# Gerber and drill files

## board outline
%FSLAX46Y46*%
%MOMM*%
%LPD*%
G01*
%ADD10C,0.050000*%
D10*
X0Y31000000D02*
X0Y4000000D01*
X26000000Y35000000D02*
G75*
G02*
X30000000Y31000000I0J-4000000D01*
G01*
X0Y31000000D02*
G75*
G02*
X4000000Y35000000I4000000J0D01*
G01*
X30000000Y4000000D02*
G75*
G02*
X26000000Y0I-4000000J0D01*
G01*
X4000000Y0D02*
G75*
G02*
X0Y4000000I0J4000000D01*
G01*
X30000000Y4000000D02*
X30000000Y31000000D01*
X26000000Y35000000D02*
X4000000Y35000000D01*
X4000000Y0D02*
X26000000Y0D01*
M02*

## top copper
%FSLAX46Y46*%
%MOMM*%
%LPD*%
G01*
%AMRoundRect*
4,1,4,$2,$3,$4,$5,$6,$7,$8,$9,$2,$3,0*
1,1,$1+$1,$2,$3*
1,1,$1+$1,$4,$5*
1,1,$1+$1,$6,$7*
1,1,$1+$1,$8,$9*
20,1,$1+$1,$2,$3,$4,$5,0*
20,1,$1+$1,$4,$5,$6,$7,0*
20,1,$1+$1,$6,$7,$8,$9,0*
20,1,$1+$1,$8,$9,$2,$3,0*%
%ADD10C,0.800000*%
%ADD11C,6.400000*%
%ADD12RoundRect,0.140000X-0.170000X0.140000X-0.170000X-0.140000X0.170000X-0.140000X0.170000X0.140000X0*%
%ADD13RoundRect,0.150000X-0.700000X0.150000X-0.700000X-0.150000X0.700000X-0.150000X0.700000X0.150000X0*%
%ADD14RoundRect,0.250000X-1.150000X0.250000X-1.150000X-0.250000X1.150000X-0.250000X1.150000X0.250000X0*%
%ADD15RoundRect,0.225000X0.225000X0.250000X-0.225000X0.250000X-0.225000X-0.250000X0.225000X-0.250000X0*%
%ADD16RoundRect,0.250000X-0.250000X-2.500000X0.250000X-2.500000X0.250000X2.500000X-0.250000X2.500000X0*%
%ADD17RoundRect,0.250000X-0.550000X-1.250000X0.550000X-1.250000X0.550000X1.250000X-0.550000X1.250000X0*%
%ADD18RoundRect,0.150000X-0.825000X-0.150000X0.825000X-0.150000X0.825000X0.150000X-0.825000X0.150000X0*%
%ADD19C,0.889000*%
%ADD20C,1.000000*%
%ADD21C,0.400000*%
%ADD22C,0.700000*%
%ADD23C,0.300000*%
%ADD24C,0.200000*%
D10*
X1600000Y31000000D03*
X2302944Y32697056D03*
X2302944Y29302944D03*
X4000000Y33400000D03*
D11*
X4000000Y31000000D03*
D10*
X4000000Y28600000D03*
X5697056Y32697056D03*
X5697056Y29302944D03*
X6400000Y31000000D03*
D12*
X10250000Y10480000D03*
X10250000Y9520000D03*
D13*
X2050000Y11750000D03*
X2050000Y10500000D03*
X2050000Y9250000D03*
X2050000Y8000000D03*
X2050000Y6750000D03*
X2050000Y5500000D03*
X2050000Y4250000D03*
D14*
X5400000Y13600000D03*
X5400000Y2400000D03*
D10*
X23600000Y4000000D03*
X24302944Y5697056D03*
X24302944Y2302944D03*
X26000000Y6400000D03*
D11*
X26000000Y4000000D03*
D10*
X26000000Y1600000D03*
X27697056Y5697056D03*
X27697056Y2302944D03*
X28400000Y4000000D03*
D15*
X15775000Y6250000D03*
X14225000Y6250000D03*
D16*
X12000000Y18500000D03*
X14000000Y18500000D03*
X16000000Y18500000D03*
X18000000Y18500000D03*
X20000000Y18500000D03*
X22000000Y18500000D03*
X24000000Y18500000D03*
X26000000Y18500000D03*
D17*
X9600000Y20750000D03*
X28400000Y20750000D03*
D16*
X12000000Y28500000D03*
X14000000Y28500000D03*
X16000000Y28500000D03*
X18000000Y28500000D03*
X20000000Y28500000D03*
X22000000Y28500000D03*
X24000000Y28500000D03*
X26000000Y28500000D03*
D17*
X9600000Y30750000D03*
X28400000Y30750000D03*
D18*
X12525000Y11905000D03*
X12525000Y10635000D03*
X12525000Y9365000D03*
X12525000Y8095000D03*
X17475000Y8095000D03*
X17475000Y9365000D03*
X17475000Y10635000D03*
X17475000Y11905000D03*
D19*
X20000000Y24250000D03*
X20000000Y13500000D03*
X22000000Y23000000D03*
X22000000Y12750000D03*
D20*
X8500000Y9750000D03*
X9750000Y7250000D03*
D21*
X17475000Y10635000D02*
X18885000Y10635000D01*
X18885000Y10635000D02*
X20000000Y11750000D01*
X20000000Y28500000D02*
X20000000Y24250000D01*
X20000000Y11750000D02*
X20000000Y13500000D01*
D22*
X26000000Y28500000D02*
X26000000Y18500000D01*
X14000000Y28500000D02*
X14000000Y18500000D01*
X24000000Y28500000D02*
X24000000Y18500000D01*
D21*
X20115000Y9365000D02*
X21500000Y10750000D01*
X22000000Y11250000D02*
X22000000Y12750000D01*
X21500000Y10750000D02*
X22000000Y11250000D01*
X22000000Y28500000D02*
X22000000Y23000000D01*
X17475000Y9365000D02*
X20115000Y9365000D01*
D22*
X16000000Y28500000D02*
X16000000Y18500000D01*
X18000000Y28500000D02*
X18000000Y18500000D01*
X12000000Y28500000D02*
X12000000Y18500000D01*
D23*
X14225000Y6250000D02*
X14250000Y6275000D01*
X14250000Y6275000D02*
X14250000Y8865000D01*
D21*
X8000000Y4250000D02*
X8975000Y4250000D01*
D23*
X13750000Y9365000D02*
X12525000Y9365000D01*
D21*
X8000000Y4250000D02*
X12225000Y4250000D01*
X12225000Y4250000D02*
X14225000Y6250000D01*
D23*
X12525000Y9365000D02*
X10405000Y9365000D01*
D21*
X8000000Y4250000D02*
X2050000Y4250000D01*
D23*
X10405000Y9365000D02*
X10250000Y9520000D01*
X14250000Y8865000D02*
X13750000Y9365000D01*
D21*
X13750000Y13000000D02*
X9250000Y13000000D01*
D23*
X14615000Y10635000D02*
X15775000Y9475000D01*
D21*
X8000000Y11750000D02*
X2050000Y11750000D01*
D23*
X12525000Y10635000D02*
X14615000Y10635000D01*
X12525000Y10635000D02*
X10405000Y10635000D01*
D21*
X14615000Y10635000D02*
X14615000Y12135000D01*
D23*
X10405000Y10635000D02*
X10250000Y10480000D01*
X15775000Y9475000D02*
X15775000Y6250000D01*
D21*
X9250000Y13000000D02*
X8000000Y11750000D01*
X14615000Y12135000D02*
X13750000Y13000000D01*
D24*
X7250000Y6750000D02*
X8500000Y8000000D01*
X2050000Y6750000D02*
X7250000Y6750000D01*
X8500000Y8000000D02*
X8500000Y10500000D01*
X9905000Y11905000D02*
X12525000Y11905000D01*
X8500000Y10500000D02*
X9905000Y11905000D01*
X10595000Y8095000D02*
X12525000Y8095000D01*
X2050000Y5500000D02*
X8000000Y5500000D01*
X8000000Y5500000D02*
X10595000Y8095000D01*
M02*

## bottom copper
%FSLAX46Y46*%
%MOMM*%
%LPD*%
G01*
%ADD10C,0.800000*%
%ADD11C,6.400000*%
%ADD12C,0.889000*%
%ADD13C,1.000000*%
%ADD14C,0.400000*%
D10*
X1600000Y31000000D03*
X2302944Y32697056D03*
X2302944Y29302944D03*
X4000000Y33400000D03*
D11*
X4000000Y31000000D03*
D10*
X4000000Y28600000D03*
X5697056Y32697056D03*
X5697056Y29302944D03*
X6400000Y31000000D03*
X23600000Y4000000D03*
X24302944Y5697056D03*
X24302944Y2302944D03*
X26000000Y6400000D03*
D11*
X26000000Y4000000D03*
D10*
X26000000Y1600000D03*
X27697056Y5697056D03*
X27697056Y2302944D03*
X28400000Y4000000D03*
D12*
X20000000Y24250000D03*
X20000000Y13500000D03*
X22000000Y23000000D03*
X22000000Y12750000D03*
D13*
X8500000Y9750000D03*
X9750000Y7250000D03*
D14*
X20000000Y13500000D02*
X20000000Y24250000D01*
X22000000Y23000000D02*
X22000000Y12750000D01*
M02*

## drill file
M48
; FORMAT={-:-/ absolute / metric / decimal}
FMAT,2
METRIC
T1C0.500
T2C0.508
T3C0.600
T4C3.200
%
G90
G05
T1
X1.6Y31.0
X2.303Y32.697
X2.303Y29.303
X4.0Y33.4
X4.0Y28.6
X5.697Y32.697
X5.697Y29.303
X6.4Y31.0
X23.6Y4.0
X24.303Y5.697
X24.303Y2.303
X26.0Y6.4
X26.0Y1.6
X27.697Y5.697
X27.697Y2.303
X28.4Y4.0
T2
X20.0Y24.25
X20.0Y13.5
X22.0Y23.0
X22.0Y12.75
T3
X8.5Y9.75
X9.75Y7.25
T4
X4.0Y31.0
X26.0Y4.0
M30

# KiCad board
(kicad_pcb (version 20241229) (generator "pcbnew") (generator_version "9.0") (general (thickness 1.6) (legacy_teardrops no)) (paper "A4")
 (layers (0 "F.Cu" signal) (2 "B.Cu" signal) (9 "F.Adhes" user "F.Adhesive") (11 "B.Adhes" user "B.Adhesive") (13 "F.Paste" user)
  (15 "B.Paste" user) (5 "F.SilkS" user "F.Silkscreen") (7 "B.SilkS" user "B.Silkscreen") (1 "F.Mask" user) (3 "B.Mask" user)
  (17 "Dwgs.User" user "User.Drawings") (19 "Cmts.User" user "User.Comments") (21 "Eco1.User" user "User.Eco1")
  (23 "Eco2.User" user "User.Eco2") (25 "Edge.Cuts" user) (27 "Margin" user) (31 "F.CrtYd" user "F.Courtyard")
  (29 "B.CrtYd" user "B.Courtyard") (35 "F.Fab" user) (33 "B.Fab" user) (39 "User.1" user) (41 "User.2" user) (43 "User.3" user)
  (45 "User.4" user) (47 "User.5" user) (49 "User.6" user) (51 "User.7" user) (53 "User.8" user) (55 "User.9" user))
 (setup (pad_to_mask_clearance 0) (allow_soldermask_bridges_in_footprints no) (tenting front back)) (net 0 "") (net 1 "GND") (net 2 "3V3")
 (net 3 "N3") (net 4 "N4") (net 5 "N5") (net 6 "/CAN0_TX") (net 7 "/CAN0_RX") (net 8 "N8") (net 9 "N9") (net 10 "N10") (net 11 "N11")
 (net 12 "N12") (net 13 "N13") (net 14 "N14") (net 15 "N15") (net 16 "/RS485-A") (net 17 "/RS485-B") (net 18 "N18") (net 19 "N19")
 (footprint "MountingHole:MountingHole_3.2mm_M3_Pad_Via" (layer "F.Cu") (at 4 -31)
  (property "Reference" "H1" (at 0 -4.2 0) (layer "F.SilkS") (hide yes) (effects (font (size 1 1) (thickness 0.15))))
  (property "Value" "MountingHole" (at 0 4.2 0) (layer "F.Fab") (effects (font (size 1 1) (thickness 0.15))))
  (pad "1" thru_hole circle (at -2.4 0) (size 0.8 0.8) (drill 0.5) (layers "*.Cu" "*.Mask") (remove_unused_layers no) (zone_connect 2))
  (pad "1" thru_hole circle (at -1.697056 -1.697056) (size 0.8 0.8) (drill 0.5) (layers "*.Cu" "*.Mask") (remove_unused_layers no)
   (zone_connect 2))
  (pad "1" thru_hole circle (at -1.697056 1.697056) (size 0.8 0.8) (drill 0.5) (layers "*.Cu" "*.Mask") (remove_unused_layers no)
   (zone_connect 2))
  (pad "1" thru_hole circle (at 0 -2.4) (size 0.8 0.8) (drill 0.5) (layers "*.Cu" "*.Mask") (remove_unused_layers no) (zone_connect 2))
  (pad "1" thru_hole circle (at 0 0) (size 6.4 6.4) (drill 3.2) (layers "*.Cu" "*.Mask") (remove_unused_layers no))
  (pad "1" thru_hole circle (at 0 2.4) (size 0.8 0.8) (drill 0.5) (layers "*.Cu" "*.Mask") (remove_unused_layers no) (zone_connect 2))
  (pad "1" thru_hole circle (at 1.697056 -1.697056) (size 0.8 0.8) (drill 0.5) (layers "*.Cu" "*.Mask") (remove_unused_layers no)
   (zone_connect 2))
  (pad "1" thru_hole circle (at 1.697056 1.697056) (size 0.8 0.8) (drill 0.5) (layers "*.Cu" "*.Mask") (remove_unused_layers no)
   (zone_connect 2))
  (pad "1" thru_hole circle (at 2.4 0) (size 0.8 0.8) (drill 0.5) (layers "*.Cu" "*.Mask") (remove_unused_layers no) (zone_connect 2)))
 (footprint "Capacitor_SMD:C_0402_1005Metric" (layer "F.Cu") (at 10.25 -10 -90)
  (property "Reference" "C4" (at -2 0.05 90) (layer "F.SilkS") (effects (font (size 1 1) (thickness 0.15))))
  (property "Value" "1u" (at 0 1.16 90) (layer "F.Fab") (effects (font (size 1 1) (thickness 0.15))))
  (pad "1" smd roundrect (at -0.48 0 270) (size 0.56 0.62) (layers "F.Cu" "F.Mask" "F.Paste") (roundrect_rratio 0.25) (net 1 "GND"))
  (pad "2" smd roundrect (at 0.48 0 270) (size 0.56 0.62) (layers "F.Cu" "F.Mask" "F.Paste") (roundrect_rratio 0.25) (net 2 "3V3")))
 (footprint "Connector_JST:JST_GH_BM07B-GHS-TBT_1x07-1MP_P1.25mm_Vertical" (layer "F.Cu") (at 4 -8 -90)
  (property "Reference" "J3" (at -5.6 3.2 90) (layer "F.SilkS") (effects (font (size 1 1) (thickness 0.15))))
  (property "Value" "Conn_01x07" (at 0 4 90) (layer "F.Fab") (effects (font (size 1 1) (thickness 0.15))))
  (pad "1" smd roundrect (at -3.75 1.95 270) (size 0.6 1.7) (layers "F.Cu" "F.Mask" "F.Paste") (roundrect_rratio 0.25) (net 1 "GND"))
  (pad "2" smd roundrect (at -2.5 1.95 270) (size 0.6 1.7) (layers "F.Cu" "F.Mask" "F.Paste") (roundrect_rratio 0.25) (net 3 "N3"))
  (pad "3" smd roundrect (at -1.25 1.95 270) (size 0.6 1.7) (layers "F.Cu" "F.Mask" "F.Paste") (roundrect_rratio 0.25) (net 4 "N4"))
  (pad "4" smd roundrect (at 0 1.95 270) (size 0.6 1.7) (layers "F.Cu" "F.Mask" "F.Paste") (roundrect_rratio 0.25) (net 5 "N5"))
  (pad "5" smd roundrect (at 1.25 1.95 270) (size 0.6 1.7) (layers "F.Cu" "F.Mask" "F.Paste") (roundrect_rratio 0.25) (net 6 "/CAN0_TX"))
  (pad "6" smd roundrect (at 2.5 1.95 270) (size 0.6 1.7) (layers "F.Cu" "F.Mask" "F.Paste") (roundrect_rratio 0.25) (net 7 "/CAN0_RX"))
  (pad "7" smd roundrect (at 3.75 1.95 270) (size 0.6 1.7) (layers "F.Cu" "F.Mask" "F.Paste") (roundrect_rratio 0.25) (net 2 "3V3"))
  (pad "MP" smd roundrect (at -5.6 -1.4 270) (size 1 2.8) (layers "F.Cu" "F.Mask" "F.Paste") (roundrect_rratio 0.25))
  (pad "MP" smd roundrect (at 5.6 -1.4 270) (size 1 2.8) (layers "F.Cu" "F.Mask" "F.Paste") (roundrect_rratio 0.25)))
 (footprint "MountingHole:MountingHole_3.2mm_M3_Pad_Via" (layer "F.Cu") (at 26 -4)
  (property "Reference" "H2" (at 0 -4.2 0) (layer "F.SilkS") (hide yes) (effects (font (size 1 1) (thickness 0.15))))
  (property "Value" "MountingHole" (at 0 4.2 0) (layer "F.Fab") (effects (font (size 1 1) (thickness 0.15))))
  (pad "1" thru_hole circle (at -2.4 0) (size 0.8 0.8) (drill 0.5) (layers "*.Cu" "*.Mask") (remove_unused_layers no) (zone_connect 2))
  (pad "1" thru_hole circle (at -1.697056 -1.697056) (size 0.8 0.8) (drill 0.5) (layers "*.Cu" "*.Mask") (remove_unused_layers no)
   (zone_connect 2))
  (pad "1" thru_hole circle (at -1.697056 1.697056) (size 0.8 0.8) (drill 0.5) (layers "*.Cu" "*.Mask") (remove_unused_layers no)
   (zone_connect 2))
  (pad "1" thru_hole circle (at 0 -2.4) (size 0.8 0.8) (drill 0.5) (layers "*.Cu" "*.Mask") (remove_unused_layers no) (zone_connect 2))
  (pad "1" thru_hole circle (at 0 0) (size 6.4 6.4) (drill 3.2) (layers "*.Cu" "*.Mask") (remove_unused_layers no))
  (pad "1" thru_hole circle (at 0 2.4) (size 0.8 0.8) (drill 0.5) (layers "*.Cu" "*.Mask") (remove_unused_layers no) (zone_connect 2))
  (pad "1" thru_hole circle (at 1.697056 -1.697056) (size 0.8 0.8) (drill 0.5) (layers "*.Cu" "*.Mask") (remove_unused_layers no)
   (zone_connect 2))
  (pad "1" thru_hole circle (at 1.697056 1.697056) (size 0.8 0.8) (drill 0.5) (layers "*.Cu" "*.Mask") (remove_unused_layers no)
   (zone_connect 2))
  (pad "1" thru_hole circle (at 2.4 0) (size 0.8 0.8) (drill 0.5) (layers "*.Cu" "*.Mask") (remove_unused_layers no) (zone_connect 2)))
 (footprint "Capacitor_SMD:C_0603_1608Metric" (layer "F.Cu") (at 15 -6.25 180)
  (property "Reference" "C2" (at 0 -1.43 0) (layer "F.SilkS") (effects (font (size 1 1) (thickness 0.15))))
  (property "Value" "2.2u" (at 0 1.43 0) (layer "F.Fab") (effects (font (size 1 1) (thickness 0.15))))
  (pad "1" smd roundrect (at -0.775 0 180) (size 0.9 0.95) (layers "F.Cu" "F.Mask" "F.Paste") (roundrect_rratio 0.25) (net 1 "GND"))
  (pad "2" smd roundrect (at 0.775 0 180) (size 0.9 0.95) (layers "F.Cu" "F.Mask" "F.Paste") (roundrect_rratio 0.25) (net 2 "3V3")))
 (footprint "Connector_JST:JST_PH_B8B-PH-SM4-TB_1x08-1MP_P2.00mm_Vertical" (layer "F.Cu") (at 19 -19)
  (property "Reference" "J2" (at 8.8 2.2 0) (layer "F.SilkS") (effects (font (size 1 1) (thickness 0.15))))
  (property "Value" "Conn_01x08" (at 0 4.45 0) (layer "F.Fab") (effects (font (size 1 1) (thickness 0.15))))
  (pad "1" smd roundrect (at -7 0.5) (size 1 5.5) (layers "F.Cu" "F.Mask" "F.Paste") (roundrect_rratio 0.25) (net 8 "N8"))
  (pad "2" smd roundrect (at -5 0.5) (size 1 5.5) (layers "F.Cu" "F.Mask" "F.Paste") (roundrect_rratio 0.25) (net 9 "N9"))
  (pad "3" smd roundrect (at -3 0.5) (size 1 5.5) (layers "F.Cu" "F.Mask" "F.Paste") (roundrect_rratio 0.25) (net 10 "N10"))
  (pad "4" smd roundrect (at -1 0.5) (size 1 5.5) (layers "F.Cu" "F.Mask" "F.Paste") (roundrect_rratio 0.25) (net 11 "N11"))
  (pad "5" smd roundrect (at 1 0.5) (size 1 5.5) (layers "F.Cu" "F.Mask" "F.Paste") (roundrect_rratio 0.25) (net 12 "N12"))
  (pad "6" smd roundrect (at 3 0.5) (size 1 5.5) (layers "F.Cu" "F.Mask" "F.Paste") (roundrect_rratio 0.25) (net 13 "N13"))
  (pad "7" smd roundrect (at 5 0.5) (size 1 5.5) (layers "F.Cu" "F.Mask" "F.Paste") (roundrect_rratio 0.25) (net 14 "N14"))
  (pad "8" smd roundrect (at 7 0.5) (size 1 5.5) (layers "F.Cu" "F.Mask" "F.Paste") (roundrect_rratio 0.25) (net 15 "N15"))
  (pad "MP" smd roundrect (at -9.4 -1.75) (size 1.6 3) (layers "F.Cu" "F.Mask" "F.Paste") (roundrect_rratio 0.15625))
  (pad "MP" smd roundrect (at 9.4 -1.75) (size 1.6 3) (layers "F.Cu" "F.Mask" "F.Paste") (roundrect_rratio 0.15625)))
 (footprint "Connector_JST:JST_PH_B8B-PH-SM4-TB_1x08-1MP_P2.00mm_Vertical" (layer "F.Cu") (at 19 -29)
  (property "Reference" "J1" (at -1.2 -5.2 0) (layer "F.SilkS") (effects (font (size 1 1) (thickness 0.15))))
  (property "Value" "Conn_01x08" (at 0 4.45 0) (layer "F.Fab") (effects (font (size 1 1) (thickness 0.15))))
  (pad "1" smd roundrect (at -7 0.5) (size 1 5.5) (layers "F.Cu" "F.Mask" "F.Paste") (roundrect_rratio 0.25) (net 8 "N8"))
  (pad "2" smd roundrect (at -5 0.5) (size 1 5.5) (layers "F.Cu" "F.Mask" "F.Paste") (roundrect_rratio 0.25) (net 9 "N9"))
  (pad "3" smd roundrect (at -3 0.5) (size 1 5.5) (layers "F.Cu" "F.Mask" "F.Paste") (roundrect_rratio 0.25) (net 10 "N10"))
  (pad "4" smd roundrect (at -1 0.5) (size 1 5.5) (layers "F.Cu" "F.Mask" "F.Paste") (roundrect_rratio 0.25) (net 11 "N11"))
  (pad "5" smd roundrect (at 1 0.5) (size 1 5.5) (layers "F.Cu" "F.Mask" "F.Paste") (roundrect_rratio 0.25) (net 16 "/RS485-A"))
  (pad "6" smd roundrect (at 3 0.5) (size 1 5.5) (layers "F.Cu" "F.Mask" "F.Paste") (roundrect_rratio 0.25) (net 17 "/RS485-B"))
  (pad "7" smd roundrect (at 5 0.5) (size 1 5.5) (layers "F.Cu" "F.Mask" "F.Paste") (roundrect_rratio 0.25) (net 14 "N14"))
  (pad "8" smd roundrect (at 7 0.5) (size 1 5.5) (layers "F.Cu" "F.Mask" "F.Paste") (roundrect_rratio 0.25) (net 15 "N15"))
  (pad "MP" smd roundrect (at -9.4 -1.75) (size 1.6 3) (layers "F.Cu" "F.Mask" "F.Paste") (roundrect_rratio 0.15625))
  (pad "MP" smd roundrect (at 9.4 -1.75) (size 1.6 3) (layers "F.Cu" "F.Mask" "F.Paste") (roundrect_rratio 0.15625)))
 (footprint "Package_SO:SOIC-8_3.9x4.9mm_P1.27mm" (layer "F.Cu") (at 15 -10)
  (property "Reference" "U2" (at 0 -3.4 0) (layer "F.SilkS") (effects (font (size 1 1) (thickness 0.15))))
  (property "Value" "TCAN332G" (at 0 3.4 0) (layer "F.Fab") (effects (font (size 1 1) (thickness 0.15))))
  (pad "1" smd roundrect (at -2.475 -1.905) (size 1.95 0.6) (layers "F.Cu" "F.Mask" "F.Paste") (roundrect_rratio 0.25) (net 6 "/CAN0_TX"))
  (pad "2" smd roundrect (at -2.475 -0.635) (size 1.95 0.6) (layers "F.Cu" "F.Mask" "F.Paste") (roundrect_rratio 0.25) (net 1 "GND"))
  (pad "3" smd roundrect (at -2.475 0.635) (size 1.95 0.6) (layers "F.Cu" "F.Mask" "F.Paste") (roundrect_rratio 0.25) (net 2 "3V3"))
  (pad "4" smd roundrect (at -2.475 1.905) (size 1.95 0.6) (layers "F.Cu" "F.Mask" "F.Paste") (roundrect_rratio 0.25) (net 7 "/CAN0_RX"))
  (pad "5" smd roundrect (at 2.475 1.905) (size 1.95 0.6) (layers "F.Cu" "F.Mask" "F.Paste") (roundrect_rratio 0.25) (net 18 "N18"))
  (pad "6" smd roundrect (at 2.475 0.635) (size 1.95 0.6) (layers "F.Cu" "F.Mask" "F.Paste") (roundrect_rratio 0.25) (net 17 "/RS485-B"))
  (pad "7" smd roundrect (at 2.475 -0.635) (size 1.95 0.6) (layers "F.Cu" "F.Mask" "F.Paste") (roundrect_rratio 0.25) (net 16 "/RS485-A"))
  (pad "8" smd roundrect (at 2.475 -1.905) (size 1.95 0.6) (layers "F.Cu" "F.Mask" "F.Paste") (roundrect_rratio 0.25) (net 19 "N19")))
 (gr_line (start 0 -31) (end 0 -4) (stroke (width 0.05) (type default)) (layer "Edge.Cuts"))
 (gr_arc (start 26 -35) (mid 28.828427 -33.828427) (end 30 -31) (stroke (width 0.05) (type default)) (layer "Edge.Cuts"))
 (gr_arc (start 0 -31) (mid 1.171573 -33.828427) (end 4 -35) (stroke (width 0.05) (type default)) (layer "Edge.Cuts"))
 (gr_arc (start 30 -4) (mid 28.828427 -1.171573) (end 26 0) (stroke (width 0.05) (type default)) (layer "Edge.Cuts"))
 (gr_arc (start 4 0) (mid 1.171573 -1.171573) (end 0 -4) (stroke (width 0.05) (type default)) (layer "Edge.Cuts"))
 (gr_line (start 30 -4) (end 30 -31) (stroke (width 0.05) (type default)) (layer "Edge.Cuts"))
 (gr_line (start 26 -35) (end 4 -35) (stroke (width 0.05) (type default)) (layer "Edge.Cuts"))
 (gr_line (start 4 0) (end 26 0) (stroke (width 0.05) (type default)) (layer "Edge.Cuts"))
 (segment (start 17.475 -10.635) (end 18.885 -10.635) (width 0.4) (layer "F.Cu") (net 16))
 (segment (start 18.885 -10.635) (end 20 -11.75) (width 0.4) (layer "F.Cu") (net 16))
 (segment (start 20 -28.5) (end 20 -24.25) (width 0.4) (layer "F.Cu") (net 16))
 (segment (start 20 -11.75) (end 20 -13.5) (width 0.4) (layer "F.Cu") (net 16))
 (via (at 20 -24.25) (size 0.889) (drill 0.508) (layers "F.Cu" "B.Cu") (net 16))
 (via (at 20 -13.5) (size 0.889) (drill 0.508) (layers "F.Cu" "B.Cu") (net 16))
 (segment (start 20 -13.5) (end 20 -24.25) (width 0.4) (layer "B.Cu") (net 16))
 (segment (start 26 -28.5) (end 26 -18.5) (width 0.7) (layer "F.Cu") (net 15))
 (segment (start 14 -28.5) (end 14 -18.5) (width 0.7) (layer "F.Cu") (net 9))
 (segment (start 24 -28.5) (end 24 -18.5) (width 0.7) (layer "F.Cu") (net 14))
 (segment (start 20.115 -9.365) (end 21.5 -10.75) (width 0.4) (layer "F.Cu") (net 17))
 (segment (start 22 -11.25) (end 22 -12.75) (width 0.4) (layer "F.Cu") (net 17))
 (segment (start 21.5 -10.75) (end 22 -11.25) (width 0.4) (layer "F.Cu") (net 17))
 (segment (start 22 -28.5) (end 22 -23) (width 0.4) (layer "F.Cu") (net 17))
 (segment (start 17.475 -9.365) (end 20.115 -9.365) (width 0.4) (layer "F.Cu") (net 17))
 (via (at 22 -23) (size 0.889) (drill 0.508) (layers "F.Cu" "B.Cu") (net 17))
 (via (at 22 -12.75) (size 0.889) (drill 0.508) (layers "F.Cu" "B.Cu") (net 17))
 (segment (start 22 -23) (end 22 -12.75) (width 0.4) (layer "B.Cu") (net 17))
 (segment (start 16 -28.5) (end 16 -18.5) (width 0.7) (layer "F.Cu") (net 10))
 (segment (start 18 -28.5) (end 18 -18.5) (width 0.7) (layer "F.Cu") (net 11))
 (segment (start 12 -28.5) (end 12 -18.5) (width 0.7) (layer "F.Cu") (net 8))
 (segment (start 14.225 -6.25) (end 14.25 -6.275) (width 0.3) (layer "F.Cu") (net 2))
 (segment (start 14.25 -6.275) (end 14.25 -8.865) (width 0.3) (layer "F.Cu") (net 2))
 (segment (start 8 -4.25) (end 8.975 -4.25) (width 0.4) (layer "F.Cu") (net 2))
 (segment (start 13.75 -9.365) (end 12.525 -9.365) (width 0.3) (layer "F.Cu") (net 2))
 (segment (start 8 -4.25) (end 12.225 -4.25) (width 0.4) (layer "F.Cu") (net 2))
 (segment (start 12.225 -4.25) (end 14.225 -6.25) (width 0.4) (layer "F.Cu") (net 2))
 (segment (start 12.525 -9.365) (end 10.405 -9.365) (width 0.3) (layer "F.Cu") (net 2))
 (segment (start 8 -4.25) (end 2.05 -4.25) (width 0.4) (layer "F.Cu") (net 2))
 (segment (start 10.405 -9.365) (end 10.25 -9.52) (width 0.3) (layer "F.Cu") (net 2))
 (segment (start 14.25 -8.865) (end 13.75 -9.365) (width 0.3) (layer "F.Cu") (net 2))
 (segment (start 13.75 -13) (end 9.25 -13) (width 0.4) (layer "F.Cu") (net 1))
 (segment (start 14.615 -10.635) (end 15.775 -9.475) (width 0.3) (layer "F.Cu") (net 1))
 (segment (start 8 -11.75) (end 2.05 -11.75) (width 0.4) (layer "F.Cu") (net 1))
 (segment (start 12.525 -10.635) (end 14.615 -10.635) (width 0.3) (layer "F.Cu") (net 1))
 (segment (start 12.525 -10.635) (end 10.405 -10.635) (width 0.3) (layer "F.Cu") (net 1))
 (segment (start 14.615 -10.635) (end 14.615 -12.135) (width 0.4) (layer "F.Cu") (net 1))
 (segment (start 10.405 -10.635) (end 10.25 -10.48) (width 0.3) (layer "F.Cu") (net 1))
 (segment (start 15.775 -9.475) (end 15.775 -6.25) (width 0.3) (layer "F.Cu") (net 1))
 (segment (start 9.25 -13) (end 8 -11.75) (width 0.4) (layer "F.Cu") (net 1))
 (segment (start 14.615 -12.135) (end 13.75 -13) (width 0.4) (layer "F.Cu") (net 1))
 (segment (start 7.25 -6.75) (end 8.5 -8) (width 0.2) (layer "F.Cu") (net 6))
 (segment (start 2.05 -6.75) (end 7.25 -6.75) (width 0.2) (layer "F.Cu") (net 6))
 (segment (start 8.5 -8) (end 8.5 -10.5) (width 0.2) (layer "F.Cu") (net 6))
 (segment (start 9.905 -11.905) (end 12.525 -11.905) (width 0.2) (layer "F.Cu") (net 6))
 (segment (start 8.5 -10.5) (end 9.905 -11.905) (width 0.2) (layer "F.Cu") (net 6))
 (via (at 8.5 -9.75) (size 1) (drill 0.6) (layers "F.Cu" "B.Cu") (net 6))
 (segment (start 10.595 -8.095) (end 12.525 -8.095) (width 0.2) (layer "F.Cu") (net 7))
 (segment (start 2.05 -5.5) (end 8 -5.5) (width 0.2) (layer "F.Cu") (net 7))
 (segment (start 8 -5.5) (end 10.595 -8.095) (width 0.2) (layer "F.Cu") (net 7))
 (via (at 9.75 -7.25) (size 1) (drill 0.6) (layers "F.Cu" "B.Cu") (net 7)))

